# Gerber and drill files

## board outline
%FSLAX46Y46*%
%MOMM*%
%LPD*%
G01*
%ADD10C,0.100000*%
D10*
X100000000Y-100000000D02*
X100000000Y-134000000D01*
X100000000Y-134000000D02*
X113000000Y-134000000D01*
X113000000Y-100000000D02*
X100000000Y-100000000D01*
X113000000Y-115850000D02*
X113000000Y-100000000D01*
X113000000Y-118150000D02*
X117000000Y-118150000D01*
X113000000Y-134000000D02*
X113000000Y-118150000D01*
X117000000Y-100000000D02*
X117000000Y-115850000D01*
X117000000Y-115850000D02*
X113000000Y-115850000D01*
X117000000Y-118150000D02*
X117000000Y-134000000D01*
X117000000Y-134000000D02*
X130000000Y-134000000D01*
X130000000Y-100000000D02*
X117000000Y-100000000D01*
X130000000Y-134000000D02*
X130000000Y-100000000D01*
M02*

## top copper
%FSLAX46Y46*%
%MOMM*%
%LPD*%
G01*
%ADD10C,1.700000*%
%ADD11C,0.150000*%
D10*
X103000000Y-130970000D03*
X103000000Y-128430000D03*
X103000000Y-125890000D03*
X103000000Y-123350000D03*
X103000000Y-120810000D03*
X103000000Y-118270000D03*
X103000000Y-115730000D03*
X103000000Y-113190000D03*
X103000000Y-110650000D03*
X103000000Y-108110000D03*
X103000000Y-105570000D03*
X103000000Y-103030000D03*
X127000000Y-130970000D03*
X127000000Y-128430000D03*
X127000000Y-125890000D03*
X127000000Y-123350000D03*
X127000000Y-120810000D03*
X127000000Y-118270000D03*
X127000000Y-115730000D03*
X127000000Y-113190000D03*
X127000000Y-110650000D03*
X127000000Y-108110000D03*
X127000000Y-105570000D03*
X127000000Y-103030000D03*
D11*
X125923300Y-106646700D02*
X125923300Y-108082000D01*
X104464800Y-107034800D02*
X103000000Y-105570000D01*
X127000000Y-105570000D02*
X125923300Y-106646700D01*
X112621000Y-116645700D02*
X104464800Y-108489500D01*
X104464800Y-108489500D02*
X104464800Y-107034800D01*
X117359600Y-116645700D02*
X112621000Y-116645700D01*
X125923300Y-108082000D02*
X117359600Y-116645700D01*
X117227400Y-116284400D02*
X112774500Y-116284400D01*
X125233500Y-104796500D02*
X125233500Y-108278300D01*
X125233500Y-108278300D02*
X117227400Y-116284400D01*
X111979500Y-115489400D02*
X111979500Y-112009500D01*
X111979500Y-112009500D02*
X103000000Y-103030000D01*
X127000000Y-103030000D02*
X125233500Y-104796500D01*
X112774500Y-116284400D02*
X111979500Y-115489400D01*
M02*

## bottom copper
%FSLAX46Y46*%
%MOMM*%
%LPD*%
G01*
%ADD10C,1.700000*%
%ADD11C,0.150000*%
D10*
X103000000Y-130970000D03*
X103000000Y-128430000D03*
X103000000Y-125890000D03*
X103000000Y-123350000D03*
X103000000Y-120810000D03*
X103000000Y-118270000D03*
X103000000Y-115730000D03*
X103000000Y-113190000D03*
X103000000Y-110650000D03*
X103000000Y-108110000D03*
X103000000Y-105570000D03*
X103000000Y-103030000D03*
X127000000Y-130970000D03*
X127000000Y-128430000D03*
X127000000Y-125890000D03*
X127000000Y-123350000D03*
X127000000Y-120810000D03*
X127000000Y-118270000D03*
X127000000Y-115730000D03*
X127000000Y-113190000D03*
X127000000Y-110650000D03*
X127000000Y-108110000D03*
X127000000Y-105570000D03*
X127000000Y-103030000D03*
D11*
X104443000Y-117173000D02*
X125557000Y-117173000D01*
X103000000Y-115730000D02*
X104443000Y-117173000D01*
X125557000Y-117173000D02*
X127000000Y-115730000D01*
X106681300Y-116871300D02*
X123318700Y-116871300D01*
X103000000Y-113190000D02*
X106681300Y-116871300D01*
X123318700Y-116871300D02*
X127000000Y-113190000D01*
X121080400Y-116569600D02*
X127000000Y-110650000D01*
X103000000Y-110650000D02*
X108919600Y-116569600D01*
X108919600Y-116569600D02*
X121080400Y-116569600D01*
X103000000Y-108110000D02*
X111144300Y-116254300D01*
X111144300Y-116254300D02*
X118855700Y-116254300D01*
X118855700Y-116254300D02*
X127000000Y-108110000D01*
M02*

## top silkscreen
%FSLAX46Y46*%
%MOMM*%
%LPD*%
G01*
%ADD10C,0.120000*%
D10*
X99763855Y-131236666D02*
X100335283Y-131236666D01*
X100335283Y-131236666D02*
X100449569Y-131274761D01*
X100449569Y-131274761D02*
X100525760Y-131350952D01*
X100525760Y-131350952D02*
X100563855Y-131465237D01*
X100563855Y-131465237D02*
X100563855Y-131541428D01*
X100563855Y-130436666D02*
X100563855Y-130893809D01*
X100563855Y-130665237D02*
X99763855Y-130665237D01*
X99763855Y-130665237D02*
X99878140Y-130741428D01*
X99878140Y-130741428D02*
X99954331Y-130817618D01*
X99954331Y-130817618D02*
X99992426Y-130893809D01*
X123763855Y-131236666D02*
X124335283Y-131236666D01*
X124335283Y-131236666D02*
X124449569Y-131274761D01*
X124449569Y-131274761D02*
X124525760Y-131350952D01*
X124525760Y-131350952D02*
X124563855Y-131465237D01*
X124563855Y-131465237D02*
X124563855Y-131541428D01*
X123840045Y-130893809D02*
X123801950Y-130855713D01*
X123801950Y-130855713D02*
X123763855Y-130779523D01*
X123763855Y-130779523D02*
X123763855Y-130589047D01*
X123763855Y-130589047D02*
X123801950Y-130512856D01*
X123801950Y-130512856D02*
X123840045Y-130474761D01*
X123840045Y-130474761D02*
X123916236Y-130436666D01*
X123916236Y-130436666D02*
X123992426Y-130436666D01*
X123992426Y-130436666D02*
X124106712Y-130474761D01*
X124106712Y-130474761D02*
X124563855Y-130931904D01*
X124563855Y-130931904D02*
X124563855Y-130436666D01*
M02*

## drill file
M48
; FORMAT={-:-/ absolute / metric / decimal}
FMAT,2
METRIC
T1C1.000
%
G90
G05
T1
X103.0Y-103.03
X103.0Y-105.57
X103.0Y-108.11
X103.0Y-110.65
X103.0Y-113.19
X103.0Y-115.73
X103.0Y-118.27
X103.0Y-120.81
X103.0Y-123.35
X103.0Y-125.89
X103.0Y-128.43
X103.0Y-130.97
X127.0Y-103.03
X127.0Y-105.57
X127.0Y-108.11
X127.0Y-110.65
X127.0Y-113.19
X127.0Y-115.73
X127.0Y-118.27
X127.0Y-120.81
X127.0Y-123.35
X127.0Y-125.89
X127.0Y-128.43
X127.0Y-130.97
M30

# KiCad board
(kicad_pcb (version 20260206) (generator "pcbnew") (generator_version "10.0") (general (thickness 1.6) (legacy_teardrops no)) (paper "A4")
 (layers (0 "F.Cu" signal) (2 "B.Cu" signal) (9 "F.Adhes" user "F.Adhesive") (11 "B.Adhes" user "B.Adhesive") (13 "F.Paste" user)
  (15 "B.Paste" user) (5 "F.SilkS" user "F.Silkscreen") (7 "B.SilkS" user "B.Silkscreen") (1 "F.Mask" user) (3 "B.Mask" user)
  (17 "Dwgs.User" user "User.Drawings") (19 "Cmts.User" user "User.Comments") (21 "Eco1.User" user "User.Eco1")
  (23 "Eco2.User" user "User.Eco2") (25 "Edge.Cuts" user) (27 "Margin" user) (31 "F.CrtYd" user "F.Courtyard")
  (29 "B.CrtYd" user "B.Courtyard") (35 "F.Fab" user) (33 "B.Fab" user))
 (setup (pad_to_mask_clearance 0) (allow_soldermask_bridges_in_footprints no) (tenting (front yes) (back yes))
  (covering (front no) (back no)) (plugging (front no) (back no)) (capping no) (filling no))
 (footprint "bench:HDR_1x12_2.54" (layer "F.Cu") (at 103 130.97 90)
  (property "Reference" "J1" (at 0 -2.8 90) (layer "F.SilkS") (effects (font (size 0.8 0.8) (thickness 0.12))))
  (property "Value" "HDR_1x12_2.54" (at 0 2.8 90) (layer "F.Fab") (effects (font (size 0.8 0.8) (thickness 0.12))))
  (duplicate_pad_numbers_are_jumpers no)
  (pad "1" thru_hole circle (at 0 0 90) (size 1.7 1.7) (drill 1) (layers "*.Cu" "*.Mask") (remove_unused_layers no) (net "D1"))
  (pad "2" thru_hole circle (at 2.54 0 90) (size 1.7 1.7) (drill 1) (layers "*.Cu" "*.Mask") (remove_unused_layers no) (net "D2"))
  (pad "3" thru_hole circle (at 5.08 0 90) (size 1.7 1.7) (drill 1) (layers "*.Cu" "*.Mask") (remove_unused_layers no) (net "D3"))
  (pad "4" thru_hole circle (at 7.62 0 90) (size 1.7 1.7) (drill 1) (layers "*.Cu" "*.Mask") (remove_unused_layers no) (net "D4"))
  (pad "5" thru_hole circle (at 10.16 0 90) (size 1.7 1.7) (drill 1) (layers "*.Cu" "*.Mask") (remove_unused_layers no) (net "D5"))
  (pad "6" thru_hole circle (at 12.7 0 90) (size 1.7 1.7) (drill 1) (layers "*.Cu" "*.Mask") (remove_unused_layers no) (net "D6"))
  (pad "7" thru_hole circle (at 15.24 0 90) (size 1.7 1.7) (drill 1) (layers "*.Cu" "*.Mask") (remove_unused_layers no) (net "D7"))
  (pad "8" thru_hole circle (at 17.78 0 90) (size 1.7 1.7) (drill 1) (layers "*.Cu" "*.Mask") (remove_unused_layers no) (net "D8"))
  (pad "9" thru_hole circle (at 20.32 0 90) (size 1.7 1.7) (drill 1) (layers "*.Cu" "*.Mask") (remove_unused_layers no) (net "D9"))
  (pad "10" thru_hole circle (at 22.86 0 90) (size 1.7 1.7) (drill 1) (layers "*.Cu" "*.Mask") (remove_unused_layers no) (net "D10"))
  (pad "11" thru_hole circle (at 25.4 0 90) (size 1.7 1.7) (drill 1) (layers "*.Cu" "*.Mask") (remove_unused_layers no) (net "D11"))
  (pad "12" thru_hole circle (at 27.94 0 90) (size 1.7 1.7) (drill 1) (layers "*.Cu" "*.Mask") (remove_unused_layers no) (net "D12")))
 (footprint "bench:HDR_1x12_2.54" (layer "F.Cu") (at 127 130.97 90)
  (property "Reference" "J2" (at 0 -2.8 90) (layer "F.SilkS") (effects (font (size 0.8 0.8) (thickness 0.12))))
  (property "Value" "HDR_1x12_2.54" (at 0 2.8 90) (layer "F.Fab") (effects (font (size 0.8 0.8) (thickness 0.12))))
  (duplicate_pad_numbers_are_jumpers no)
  (pad "1" thru_hole circle (at 0 0 90) (size 1.7 1.7) (drill 1) (layers "*.Cu" "*.Mask") (remove_unused_layers no) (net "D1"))
  (pad "2" thru_hole circle (at 2.54 0 90) (size 1.7 1.7) (drill 1) (layers "*.Cu" "*.Mask") (remove_unused_layers no) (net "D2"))
  (pad "3" thru_hole circle (at 5.08 0 90) (size 1.7 1.7) (drill 1) (layers "*.Cu" "*.Mask") (remove_unused_layers no) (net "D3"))
  (pad "4" thru_hole circle (at 7.62 0 90) (size 1.7 1.7) (drill 1) (layers "*.Cu" "*.Mask") (remove_unused_layers no) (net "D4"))
  (pad "5" thru_hole circle (at 10.16 0 90) (size 1.7 1.7) (drill 1) (layers "*.Cu" "*.Mask") (remove_unused_layers no) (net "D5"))
  (pad "6" thru_hole circle (at 12.7 0 90) (size 1.7 1.7) (drill 1) (layers "*.Cu" "*.Mask") (remove_unused_layers no) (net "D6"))
  (pad "7" thru_hole circle (at 15.24 0 90) (size 1.7 1.7) (drill 1) (layers "*.Cu" "*.Mask") (remove_unused_layers no) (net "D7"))
  (pad "8" thru_hole circle (at 17.78 0 90) (size 1.7 1.7) (drill 1) (layers "*.Cu" "*.Mask") (remove_unused_layers no) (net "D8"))
  (pad "9" thru_hole circle (at 20.32 0 90) (size 1.7 1.7) (drill 1) (layers "*.Cu" "*.Mask") (remove_unused_layers no) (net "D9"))
  (pad "10" thru_hole circle (at 22.86 0 90) (size 1.7 1.7) (drill 1) (layers "*.Cu" "*.Mask") (remove_unused_layers no) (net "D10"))
  (pad "11" thru_hole circle (at 25.4 0 90) (size 1.7 1.7) (drill 1) (layers "*.Cu" "*.Mask") (remove_unused_layers no) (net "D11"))
  (pad "12" thru_hole circle (at 27.94 0 90) (size 1.7 1.7) (drill 1) (layers "*.Cu" "*.Mask") (remove_unused_layers no) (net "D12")))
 (gr_line (start 100 100) (end 100 134) (stroke (width 0.1) (type solid)) (layer "Edge.Cuts"))
 (gr_line (start 100 134) (end 113 134) (stroke (width 0.1) (type solid)) (layer "Edge.Cuts"))
 (gr_line (start 113 100) (end 100 100) (stroke (width 0.1) (type solid)) (layer "Edge.Cuts"))
 (gr_line (start 113 115.85) (end 113 100) (stroke (width 0.1) (type solid)) (layer "Edge.Cuts"))
 (gr_line (start 113 118.15) (end 117 118.15) (stroke (width 0.1) (type solid)) (layer "Edge.Cuts"))
 (gr_line (start 113 134) (end 113 118.15) (stroke (width 0.1) (type solid)) (layer "Edge.Cuts"))
 (gr_line (start 117 100) (end 117 115.85) (stroke (width 0.1) (type solid)) (layer "Edge.Cuts"))
 (gr_line (start 117 115.85) (end 113 115.85) (stroke (width 0.1) (type solid)) (layer "Edge.Cuts"))
 (gr_line (start 117 118.15) (end 117 134) (stroke (width 0.1) (type solid)) (layer "Edge.Cuts"))
 (gr_line (start 117 134) (end 130 134) (stroke (width 0.1) (type solid)) (layer "Edge.Cuts"))
 (gr_line (start 130 100) (end 117 100) (stroke (width 0.1) (type solid)) (layer "Edge.Cuts"))
 (gr_line (start 130 134) (end 130 100) (stroke (width 0.1) (type solid)) (layer "Edge.Cuts"))
 (segment (start 104.443 117.173) (end 125.557 117.173) (width 0.15) (layer "B.Cu") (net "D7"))
 (segment (start 103 115.73) (end 104.443 117.173) (width 0.15) (layer "B.Cu") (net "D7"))
 (segment (start 125.557 117.173) (end 127 115.73) (width 0.15) (layer "B.Cu") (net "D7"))
 (segment (start 106.6813 116.8713) (end 123.3187 116.8713) (width 0.15) (layer "B.Cu") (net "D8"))
 (segment (start 103 113.19) (end 106.6813 116.8713) (width 0.15) (layer "B.Cu") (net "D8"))
 (segment (start 123.3187 116.8713) (end 127 113.19) (width 0.15) (layer "B.Cu") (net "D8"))
 (segment (start 121.0804 116.5696) (end 127 110.65) (width 0.15) (layer "B.Cu") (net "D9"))
 (segment (start 103 110.65) (end 108.9196 116.5696) (width 0.15) (layer "B.Cu") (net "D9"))
 (segment (start 108.9196 116.5696) (end 121.0804 116.5696) (width 0.15) (layer "B.Cu") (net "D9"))
 (segment (start 103 108.11) (end 111.1443 116.2543) (width 0.15) (layer "B.Cu") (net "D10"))
 (segment (start 111.1443 116.2543) (end 118.8557 116.2543) (width 0.15) (layer "B.Cu") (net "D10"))
 (segment (start 118.8557 116.2543) (end 127 108.11) (width 0.15) (layer "B.Cu") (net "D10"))
 (segment (start 125.9233 106.6467) (end 125.9233 108.082) (width 0.15) (layer "F.Cu") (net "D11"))
 (segment (start 104.4648 107.0348) (end 103 105.57) (width 0.15) (layer "F.Cu") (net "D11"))
 (segment (start 127 105.57) (end 125.9233 106.6467) (width 0.15) (layer "F.Cu") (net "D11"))
 (segment (start 112.621 116.6457) (end 104.4648 108.4895) (width 0.15) (layer "F.Cu") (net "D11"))
 (segment (start 104.4648 108.4895) (end 104.4648 107.0348) (width 0.15) (layer "F.Cu") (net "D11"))
 (segment (start 117.3596 116.6457) (end 112.621 116.6457) (width 0.15) (layer "F.Cu") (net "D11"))
 (segment (start 125.9233 108.082) (end 117.3596 116.6457) (width 0.15) (layer "F.Cu") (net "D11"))
 (segment (start 117.2274 116.2844) (end 112.7745 116.2844) (width 0.15) (layer "F.Cu") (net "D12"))
 (segment (start 125.2335 104.7965) (end 125.2335 108.2783) (width 0.15) (layer "F.Cu") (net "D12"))
 (segment (start 125.2335 108.2783) (end 117.2274 116.2844) (width 0.15) (layer "F.Cu") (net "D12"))
 (segment (start 111.9795 115.4894) (end 111.9795 112.0095) (width 0.15) (layer "F.Cu") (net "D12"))
 (segment (start 111.9795 112.0095) (end 103 103.03) (width 0.15) (layer "F.Cu") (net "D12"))
 (segment (start 127 103.03) (end 125.2335 104.7965) (width 0.15) (layer "F.Cu") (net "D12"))
 (segment (start 112.7745 116.2844) (end 111.9795 115.4894) (width 0.15) (layer "F.Cu") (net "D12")))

